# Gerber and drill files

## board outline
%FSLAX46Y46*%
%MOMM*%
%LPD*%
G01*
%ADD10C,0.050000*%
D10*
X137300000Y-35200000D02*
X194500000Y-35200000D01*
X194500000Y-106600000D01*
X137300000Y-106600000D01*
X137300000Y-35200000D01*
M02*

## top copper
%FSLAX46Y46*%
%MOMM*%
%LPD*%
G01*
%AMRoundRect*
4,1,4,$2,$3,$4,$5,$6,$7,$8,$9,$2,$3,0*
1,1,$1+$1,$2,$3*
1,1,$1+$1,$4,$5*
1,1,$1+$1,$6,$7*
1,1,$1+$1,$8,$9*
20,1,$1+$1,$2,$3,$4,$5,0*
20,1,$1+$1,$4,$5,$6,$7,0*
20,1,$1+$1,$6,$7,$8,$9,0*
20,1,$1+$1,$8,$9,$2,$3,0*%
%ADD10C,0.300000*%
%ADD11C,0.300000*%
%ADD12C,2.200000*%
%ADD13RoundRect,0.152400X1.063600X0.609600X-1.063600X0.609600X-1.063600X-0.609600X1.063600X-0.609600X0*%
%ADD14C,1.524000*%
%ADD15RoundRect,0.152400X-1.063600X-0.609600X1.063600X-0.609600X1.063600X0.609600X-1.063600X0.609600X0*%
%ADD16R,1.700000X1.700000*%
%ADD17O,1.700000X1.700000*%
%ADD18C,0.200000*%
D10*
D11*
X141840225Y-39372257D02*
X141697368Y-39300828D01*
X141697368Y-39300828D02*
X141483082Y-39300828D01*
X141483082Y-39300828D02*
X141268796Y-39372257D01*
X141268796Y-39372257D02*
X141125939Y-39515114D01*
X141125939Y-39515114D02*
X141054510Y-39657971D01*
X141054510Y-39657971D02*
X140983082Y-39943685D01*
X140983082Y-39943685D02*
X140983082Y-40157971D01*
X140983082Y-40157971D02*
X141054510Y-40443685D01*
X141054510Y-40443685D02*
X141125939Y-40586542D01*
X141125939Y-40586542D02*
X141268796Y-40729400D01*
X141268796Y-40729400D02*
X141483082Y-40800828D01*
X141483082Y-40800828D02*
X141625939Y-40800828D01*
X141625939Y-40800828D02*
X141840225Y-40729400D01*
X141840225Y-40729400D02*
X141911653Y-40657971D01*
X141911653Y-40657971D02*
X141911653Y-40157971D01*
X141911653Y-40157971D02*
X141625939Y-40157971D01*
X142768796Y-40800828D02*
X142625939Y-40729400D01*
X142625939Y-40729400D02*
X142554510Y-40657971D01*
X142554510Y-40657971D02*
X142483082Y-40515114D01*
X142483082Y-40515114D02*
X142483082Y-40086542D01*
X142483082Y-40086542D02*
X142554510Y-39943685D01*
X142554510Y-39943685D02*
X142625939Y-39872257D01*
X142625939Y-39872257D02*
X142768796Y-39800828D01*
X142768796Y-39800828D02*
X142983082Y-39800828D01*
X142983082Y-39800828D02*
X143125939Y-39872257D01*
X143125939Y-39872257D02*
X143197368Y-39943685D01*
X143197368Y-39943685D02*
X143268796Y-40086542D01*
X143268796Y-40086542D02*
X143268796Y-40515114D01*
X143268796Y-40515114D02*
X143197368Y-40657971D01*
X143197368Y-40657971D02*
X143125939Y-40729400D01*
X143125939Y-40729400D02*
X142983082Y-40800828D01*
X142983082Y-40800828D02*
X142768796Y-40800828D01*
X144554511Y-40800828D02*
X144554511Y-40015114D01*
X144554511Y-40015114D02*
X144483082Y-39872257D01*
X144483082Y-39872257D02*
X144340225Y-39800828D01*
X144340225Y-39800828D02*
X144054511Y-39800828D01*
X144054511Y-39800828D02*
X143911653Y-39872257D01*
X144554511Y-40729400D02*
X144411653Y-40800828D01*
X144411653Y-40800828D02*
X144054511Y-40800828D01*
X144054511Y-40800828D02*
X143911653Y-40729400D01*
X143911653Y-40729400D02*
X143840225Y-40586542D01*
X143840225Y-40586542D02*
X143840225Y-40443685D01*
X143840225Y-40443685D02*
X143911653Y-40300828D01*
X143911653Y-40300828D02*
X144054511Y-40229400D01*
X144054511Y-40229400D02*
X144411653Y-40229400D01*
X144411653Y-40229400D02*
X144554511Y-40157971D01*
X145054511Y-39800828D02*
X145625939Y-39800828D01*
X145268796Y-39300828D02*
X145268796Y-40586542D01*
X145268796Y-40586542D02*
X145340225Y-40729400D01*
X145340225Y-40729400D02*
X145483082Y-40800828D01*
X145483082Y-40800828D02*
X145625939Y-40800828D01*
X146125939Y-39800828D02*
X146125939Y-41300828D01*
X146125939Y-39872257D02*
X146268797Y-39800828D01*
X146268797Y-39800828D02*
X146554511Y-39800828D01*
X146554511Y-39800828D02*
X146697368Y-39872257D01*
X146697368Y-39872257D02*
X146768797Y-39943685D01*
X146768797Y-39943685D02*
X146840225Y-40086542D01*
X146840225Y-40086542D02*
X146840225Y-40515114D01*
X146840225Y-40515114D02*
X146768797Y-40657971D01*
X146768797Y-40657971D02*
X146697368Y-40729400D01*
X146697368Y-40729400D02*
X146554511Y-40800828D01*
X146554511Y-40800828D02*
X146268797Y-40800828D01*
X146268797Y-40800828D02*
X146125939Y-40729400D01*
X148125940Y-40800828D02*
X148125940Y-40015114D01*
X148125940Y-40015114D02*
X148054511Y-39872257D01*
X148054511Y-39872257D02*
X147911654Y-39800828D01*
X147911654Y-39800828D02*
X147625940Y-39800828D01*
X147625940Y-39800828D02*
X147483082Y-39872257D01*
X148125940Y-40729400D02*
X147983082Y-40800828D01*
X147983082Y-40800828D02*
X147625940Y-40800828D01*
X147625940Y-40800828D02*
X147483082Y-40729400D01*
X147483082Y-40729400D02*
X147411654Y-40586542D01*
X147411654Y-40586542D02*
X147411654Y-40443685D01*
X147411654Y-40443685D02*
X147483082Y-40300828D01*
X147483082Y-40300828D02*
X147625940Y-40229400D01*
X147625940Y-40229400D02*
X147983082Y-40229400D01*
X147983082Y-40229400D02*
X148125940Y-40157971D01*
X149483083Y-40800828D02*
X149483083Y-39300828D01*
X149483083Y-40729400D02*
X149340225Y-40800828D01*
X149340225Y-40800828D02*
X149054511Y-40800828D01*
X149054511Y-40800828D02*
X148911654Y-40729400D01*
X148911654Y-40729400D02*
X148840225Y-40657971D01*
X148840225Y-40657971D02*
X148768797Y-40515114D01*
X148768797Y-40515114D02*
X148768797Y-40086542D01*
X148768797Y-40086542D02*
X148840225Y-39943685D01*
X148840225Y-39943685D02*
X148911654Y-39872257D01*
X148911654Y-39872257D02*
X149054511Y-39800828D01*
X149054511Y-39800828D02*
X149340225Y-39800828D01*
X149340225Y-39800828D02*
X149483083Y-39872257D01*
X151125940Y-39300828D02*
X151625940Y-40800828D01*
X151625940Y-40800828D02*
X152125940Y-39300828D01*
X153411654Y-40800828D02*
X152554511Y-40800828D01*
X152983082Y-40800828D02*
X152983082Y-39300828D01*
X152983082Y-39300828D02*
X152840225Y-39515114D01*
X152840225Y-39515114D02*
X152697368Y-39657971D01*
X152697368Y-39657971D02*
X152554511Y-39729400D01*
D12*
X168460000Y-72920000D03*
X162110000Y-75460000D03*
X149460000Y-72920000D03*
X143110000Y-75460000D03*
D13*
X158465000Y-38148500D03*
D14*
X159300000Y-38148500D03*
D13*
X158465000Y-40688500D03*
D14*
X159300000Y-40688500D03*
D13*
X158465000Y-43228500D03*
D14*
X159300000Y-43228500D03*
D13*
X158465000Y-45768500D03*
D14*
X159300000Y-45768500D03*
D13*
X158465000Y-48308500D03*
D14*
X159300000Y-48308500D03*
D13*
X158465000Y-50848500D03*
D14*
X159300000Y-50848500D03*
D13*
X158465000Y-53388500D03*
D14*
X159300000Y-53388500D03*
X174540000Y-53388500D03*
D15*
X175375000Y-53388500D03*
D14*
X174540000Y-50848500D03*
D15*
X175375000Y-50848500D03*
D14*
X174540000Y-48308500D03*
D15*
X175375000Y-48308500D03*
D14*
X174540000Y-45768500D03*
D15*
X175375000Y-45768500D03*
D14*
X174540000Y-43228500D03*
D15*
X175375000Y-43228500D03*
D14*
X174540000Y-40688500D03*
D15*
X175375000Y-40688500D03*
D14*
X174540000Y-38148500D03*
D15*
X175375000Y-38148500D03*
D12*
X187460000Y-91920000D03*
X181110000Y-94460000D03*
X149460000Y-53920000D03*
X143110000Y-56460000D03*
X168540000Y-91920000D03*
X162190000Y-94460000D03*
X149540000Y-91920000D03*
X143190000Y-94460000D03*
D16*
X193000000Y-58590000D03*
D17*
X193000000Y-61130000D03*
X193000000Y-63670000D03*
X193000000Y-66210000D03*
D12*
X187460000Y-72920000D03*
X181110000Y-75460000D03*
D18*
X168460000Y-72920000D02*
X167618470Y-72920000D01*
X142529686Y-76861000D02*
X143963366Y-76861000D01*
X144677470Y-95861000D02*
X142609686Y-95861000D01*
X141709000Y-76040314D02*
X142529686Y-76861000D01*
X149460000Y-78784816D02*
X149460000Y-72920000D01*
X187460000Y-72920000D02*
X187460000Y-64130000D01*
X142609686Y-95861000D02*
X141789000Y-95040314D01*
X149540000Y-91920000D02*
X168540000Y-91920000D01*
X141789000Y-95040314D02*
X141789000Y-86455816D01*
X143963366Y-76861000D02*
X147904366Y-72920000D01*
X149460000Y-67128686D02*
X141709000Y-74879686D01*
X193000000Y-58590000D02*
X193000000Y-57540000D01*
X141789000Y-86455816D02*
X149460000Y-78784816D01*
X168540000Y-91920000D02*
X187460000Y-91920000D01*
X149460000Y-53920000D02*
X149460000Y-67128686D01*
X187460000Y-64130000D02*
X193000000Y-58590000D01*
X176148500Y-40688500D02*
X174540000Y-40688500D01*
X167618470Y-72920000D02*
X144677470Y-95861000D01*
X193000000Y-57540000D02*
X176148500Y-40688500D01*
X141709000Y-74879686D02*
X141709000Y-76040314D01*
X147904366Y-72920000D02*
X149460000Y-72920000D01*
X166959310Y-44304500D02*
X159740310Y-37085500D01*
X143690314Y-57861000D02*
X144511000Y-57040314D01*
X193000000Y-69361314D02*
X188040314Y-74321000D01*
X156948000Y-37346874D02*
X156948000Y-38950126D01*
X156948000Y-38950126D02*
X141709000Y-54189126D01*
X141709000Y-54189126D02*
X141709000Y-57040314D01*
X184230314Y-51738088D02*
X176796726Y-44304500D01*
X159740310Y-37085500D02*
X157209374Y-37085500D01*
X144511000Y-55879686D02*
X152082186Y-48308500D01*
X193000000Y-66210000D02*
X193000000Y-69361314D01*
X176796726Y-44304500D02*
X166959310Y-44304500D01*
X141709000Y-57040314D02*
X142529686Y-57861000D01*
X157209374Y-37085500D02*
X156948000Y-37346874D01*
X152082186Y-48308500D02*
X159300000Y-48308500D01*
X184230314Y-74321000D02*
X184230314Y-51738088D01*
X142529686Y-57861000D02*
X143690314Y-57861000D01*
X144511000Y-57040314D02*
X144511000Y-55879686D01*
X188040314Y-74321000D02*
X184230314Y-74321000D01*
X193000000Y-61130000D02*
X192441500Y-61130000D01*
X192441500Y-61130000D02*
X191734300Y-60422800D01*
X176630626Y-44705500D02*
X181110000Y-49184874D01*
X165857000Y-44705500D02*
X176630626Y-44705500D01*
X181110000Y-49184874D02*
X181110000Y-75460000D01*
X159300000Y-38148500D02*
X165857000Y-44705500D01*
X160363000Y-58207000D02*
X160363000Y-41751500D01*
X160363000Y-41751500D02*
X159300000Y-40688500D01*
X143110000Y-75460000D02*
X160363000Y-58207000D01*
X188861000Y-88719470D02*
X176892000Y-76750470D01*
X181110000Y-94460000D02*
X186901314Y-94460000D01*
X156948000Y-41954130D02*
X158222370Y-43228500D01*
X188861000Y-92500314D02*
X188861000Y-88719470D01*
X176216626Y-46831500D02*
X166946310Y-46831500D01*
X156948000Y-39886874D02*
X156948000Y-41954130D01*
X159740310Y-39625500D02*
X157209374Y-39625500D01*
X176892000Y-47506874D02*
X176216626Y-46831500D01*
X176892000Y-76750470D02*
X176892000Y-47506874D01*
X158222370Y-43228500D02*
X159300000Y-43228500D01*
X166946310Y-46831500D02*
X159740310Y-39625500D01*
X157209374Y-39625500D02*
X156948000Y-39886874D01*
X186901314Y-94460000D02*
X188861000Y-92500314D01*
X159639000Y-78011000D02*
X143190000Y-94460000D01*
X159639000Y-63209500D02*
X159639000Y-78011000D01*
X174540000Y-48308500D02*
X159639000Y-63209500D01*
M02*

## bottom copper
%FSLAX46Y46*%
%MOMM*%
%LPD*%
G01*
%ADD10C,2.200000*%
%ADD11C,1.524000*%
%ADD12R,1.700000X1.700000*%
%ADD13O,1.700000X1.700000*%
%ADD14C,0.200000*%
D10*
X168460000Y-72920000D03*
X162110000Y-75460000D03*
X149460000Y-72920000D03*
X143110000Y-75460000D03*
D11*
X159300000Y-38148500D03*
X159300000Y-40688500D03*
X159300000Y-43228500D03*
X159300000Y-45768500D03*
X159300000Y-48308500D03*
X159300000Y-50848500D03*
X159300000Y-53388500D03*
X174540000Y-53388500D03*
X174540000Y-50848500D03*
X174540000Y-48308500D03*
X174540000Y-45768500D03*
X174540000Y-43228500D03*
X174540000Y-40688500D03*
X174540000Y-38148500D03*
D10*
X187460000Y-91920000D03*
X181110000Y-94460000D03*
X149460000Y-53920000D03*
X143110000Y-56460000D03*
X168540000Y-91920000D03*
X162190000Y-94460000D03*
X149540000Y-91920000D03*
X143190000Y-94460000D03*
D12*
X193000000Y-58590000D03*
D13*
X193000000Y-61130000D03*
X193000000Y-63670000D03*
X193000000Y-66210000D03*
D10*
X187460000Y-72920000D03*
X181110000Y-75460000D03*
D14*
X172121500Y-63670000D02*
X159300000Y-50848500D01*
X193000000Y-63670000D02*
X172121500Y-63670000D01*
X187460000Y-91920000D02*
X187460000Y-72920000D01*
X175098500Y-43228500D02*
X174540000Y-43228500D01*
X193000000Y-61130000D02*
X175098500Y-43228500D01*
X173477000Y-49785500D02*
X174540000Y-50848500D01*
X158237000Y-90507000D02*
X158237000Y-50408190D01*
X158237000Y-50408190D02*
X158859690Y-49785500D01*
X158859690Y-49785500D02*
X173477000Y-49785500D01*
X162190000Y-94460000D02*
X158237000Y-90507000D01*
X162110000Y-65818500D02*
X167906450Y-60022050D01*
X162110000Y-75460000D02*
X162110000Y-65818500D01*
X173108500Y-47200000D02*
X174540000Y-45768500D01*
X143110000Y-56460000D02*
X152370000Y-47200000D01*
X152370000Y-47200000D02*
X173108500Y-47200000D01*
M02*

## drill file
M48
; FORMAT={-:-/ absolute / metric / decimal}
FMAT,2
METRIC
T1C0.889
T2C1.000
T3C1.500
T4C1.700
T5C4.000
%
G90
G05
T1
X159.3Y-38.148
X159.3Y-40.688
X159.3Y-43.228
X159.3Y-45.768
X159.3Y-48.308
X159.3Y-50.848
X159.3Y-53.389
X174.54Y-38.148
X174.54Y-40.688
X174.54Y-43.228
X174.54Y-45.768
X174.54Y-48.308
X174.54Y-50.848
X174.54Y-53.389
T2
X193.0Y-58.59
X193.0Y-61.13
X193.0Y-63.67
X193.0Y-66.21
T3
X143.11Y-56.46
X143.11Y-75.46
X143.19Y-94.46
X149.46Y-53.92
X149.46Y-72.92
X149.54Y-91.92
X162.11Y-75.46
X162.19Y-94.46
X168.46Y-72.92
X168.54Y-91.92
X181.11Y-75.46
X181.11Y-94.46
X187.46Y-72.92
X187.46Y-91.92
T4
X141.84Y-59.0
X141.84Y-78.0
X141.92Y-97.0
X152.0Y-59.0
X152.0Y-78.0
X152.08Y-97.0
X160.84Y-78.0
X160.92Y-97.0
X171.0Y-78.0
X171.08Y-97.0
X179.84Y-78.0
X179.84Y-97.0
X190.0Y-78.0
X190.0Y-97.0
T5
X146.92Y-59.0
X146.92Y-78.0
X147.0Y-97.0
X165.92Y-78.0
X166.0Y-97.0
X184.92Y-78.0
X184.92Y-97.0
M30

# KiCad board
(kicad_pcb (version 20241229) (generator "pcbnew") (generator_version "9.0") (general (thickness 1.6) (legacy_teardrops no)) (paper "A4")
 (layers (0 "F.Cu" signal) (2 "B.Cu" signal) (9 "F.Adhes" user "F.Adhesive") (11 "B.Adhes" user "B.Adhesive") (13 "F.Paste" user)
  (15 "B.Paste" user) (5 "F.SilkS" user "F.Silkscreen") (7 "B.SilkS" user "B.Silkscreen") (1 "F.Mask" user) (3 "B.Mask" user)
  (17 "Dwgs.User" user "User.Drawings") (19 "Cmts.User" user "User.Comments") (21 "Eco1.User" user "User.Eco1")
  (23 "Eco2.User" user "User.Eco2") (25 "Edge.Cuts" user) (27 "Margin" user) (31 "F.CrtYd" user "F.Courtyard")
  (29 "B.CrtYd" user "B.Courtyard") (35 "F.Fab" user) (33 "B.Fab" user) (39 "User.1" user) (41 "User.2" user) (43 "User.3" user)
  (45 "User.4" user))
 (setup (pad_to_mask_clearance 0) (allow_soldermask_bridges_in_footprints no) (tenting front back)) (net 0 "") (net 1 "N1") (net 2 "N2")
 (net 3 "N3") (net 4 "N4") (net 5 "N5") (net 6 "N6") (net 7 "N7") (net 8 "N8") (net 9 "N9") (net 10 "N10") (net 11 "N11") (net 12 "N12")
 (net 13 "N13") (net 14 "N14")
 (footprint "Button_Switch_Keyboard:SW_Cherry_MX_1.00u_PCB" (layer "F.Cu") (at 168.46 72.92)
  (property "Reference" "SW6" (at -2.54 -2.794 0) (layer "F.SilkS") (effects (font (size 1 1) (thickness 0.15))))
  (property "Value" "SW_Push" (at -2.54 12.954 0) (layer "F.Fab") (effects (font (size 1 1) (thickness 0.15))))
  (pad "" np_thru_hole circle (at -7.62 5.08) (size 1.7 1.7) (drill 1.7) (layers "*.Cu" "*.Mask"))
  (pad "" np_thru_hole circle (at -2.54 5.08) (size 4 4) (drill 4) (layers "*.Cu" "*.Mask"))
  (pad "" np_thru_hole circle (at 2.54 5.08) (size 1.7 1.7) (drill 1.7) (layers "*.Cu" "*.Mask"))
  (pad "1" thru_hole circle (at 0 0) (size 2.2 2.2) (drill 1.5) (layers "*.Cu" "*.Mask") (remove_unused_layers no) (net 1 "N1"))
  (pad "2" thru_hole circle (at -6.35 2.54) (size 2.2 2.2) (drill 1.5) (layers "*.Cu" "*.Mask") (remove_unused_layers no) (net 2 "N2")))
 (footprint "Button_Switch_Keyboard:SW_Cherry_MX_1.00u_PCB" (layer "F.Cu") (at 149.46 72.92)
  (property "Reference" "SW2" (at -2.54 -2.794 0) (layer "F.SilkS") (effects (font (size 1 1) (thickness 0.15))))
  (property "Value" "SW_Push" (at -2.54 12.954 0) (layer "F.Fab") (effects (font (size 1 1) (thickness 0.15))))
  (pad "" np_thru_hole circle (at -7.62 5.08) (size 1.7 1.7) (drill 1.7) (layers "*.Cu" "*.Mask"))
  (pad "" np_thru_hole circle (at -2.54 5.08) (size 4 4) (drill 4) (layers "*.Cu" "*.Mask"))
  (pad "" np_thru_hole circle (at 2.54 5.08) (size 1.7 1.7) (drill 1.7) (layers "*.Cu" "*.Mask"))
  (pad "1" thru_hole circle (at 0 0) (size 2.2 2.2) (drill 1.5) (layers "*.Cu" "*.Mask") (remove_unused_layers no) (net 1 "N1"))
  (pad "2" thru_hole circle (at -6.35 2.54) (size 2.2 2.2) (drill 1.5) (layers "*.Cu" "*.Mask") (remove_unused_layers no) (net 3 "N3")))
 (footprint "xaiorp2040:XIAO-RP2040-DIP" (layer "F.Cu") (at 166.92 45.7685)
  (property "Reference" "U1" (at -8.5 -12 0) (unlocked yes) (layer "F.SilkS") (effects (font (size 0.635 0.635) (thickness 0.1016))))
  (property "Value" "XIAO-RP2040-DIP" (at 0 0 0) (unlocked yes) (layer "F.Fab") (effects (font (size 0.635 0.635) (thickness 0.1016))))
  (pad "1" smd roundrect (at -8.455 -7.62 180) (size 2.432 1.524) (layers "F.Cu" "F.Mask") (roundrect_rratio 0.1) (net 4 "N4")
   (thermal_bridge_angle 45))
  (pad "1" thru_hole circle (at -7.62 -7.62 180) (size 1.524 1.524) (drill 0.889) (layers "*.Cu" "*.Mask") (remove_unused_layers no)
   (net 4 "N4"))
  (pad "2" smd roundrect (at -8.455 -5.08 180) (size 2.432 1.524) (layers "F.Cu" "F.Mask") (roundrect_rratio 0.1) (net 3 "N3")
   (thermal_bridge_angle 45))
  (pad "2" thru_hole circle (at -7.62 -5.08 180) (size 1.524 1.524) (drill 0.889) (layers "*.Cu" "*.Mask") (remove_unused_layers no)
   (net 3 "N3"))
  (pad "3" smd roundrect (at -8.455 -2.54 180) (size 2.432 1.524) (layers "F.Cu" "F.Mask") (roundrect_rratio 0.1) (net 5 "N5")
   (thermal_bridge_angle 45))
  (pad "3" thru_hole circle (at -7.62 -2.54 180) (size 1.524 1.524) (drill 0.889) (layers "*.Cu" "*.Mask") (remove_unused_layers no)
   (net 5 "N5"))
  (pad "4" smd roundrect (at -8.455 0 180) (size 2.432 1.524) (layers "F.Cu" "F.Mask") (roundrect_rratio 0.1) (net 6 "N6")
   (thermal_bridge_angle 45))
  (pad "4" thru_hole circle (at -7.62 0 180) (size 1.524 1.524) (drill 0.889) (layers "*.Cu" "*.Mask") (remove_unused_layers no)
   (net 6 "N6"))
  (pad "5" smd roundrect (at -8.455 2.54 180) (size 2.432 1.524) (layers "F.Cu" "F.Mask") (roundrect_rratio 0.1) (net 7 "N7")
   (thermal_bridge_angle 45))
  (pad "5" thru_hole circle (at -7.62 2.54 180) (size 1.524 1.524) (drill 0.889) (layers "*.Cu" "*.Mask") (remove_unused_layers no)
   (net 7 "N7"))
  (pad "6" smd roundrect (at -8.455 5.08 180) (size 2.432 1.524) (layers "F.Cu" "F.Mask") (roundrect_rratio 0.1) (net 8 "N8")
   (thermal_bridge_angle 45))
  (pad "6" thru_hole circle (at -7.62 5.08 180) (size 1.524 1.524) (drill 0.889) (layers "*.Cu" "*.Mask") (remove_unused_layers no)
   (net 8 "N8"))
  (pad "7" smd roundrect (at -8.455 7.62 180) (size 2.432 1.524) (layers "F.Cu" "F.Mask") (roundrect_rratio 0.1) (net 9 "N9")
   (thermal_bridge_angle 45))
  (pad "7" thru_hole circle (at -7.62 7.62 180) (size 1.524 1.524) (drill 0.889) (layers "*.Cu" "*.Mask") (remove_unused_layers no)
   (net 9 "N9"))
  (pad "8" thru_hole circle (at 7.62 7.62) (size 1.524 1.524) (drill 0.889) (layers "*.Cu" "*.Mask") (remove_unused_layers no) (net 2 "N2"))
  (pad "8" smd roundrect (at 8.455 7.62) (size 2.432 1.524) (layers "F.Cu" "F.Mask") (roundrect_rratio 0.1) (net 2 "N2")
   (thermal_bridge_angle 45))
  (pad "9" thru_hole circle (at 7.62 5.08) (size 1.524 1.524) (drill 0.889) (layers "*.Cu" "*.Mask") (remove_unused_layers no)
   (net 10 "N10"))
  (pad "9" smd roundrect (at 8.455 5.08) (size 2.432 1.524) (layers "F.Cu" "F.Mask") (roundrect_rratio 0.1) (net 10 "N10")
   (thermal_bridge_angle 45))
  (pad "10" thru_hole circle (at 7.62 2.54) (size 1.524 1.524) (drill 0.889) (layers "*.Cu" "*.Mask") (remove_unused_layers no)
   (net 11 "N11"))
  (pad "10" smd roundrect (at 8.455 2.54) (size 2.432 1.524) (layers "F.Cu" "F.Mask") (roundrect_rratio 0.1) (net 11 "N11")
   (thermal_bridge_angle 45))
  (pad "11" thru_hole circle (at 7.62 0) (size 1.524 1.524) (drill 0.889) (layers "*.Cu" "*.Mask") (remove_unused_layers no) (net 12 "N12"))
  (pad "11" smd roundrect (at 8.455 0) (size 2.432 1.524) (layers "F.Cu" "F.Mask") (roundrect_rratio 0.1) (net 12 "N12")
   (thermal_bridge_angle 45))
  (pad "12" thru_hole circle (at 7.62 -2.54) (size 1.524 1.524) (drill 0.889) (layers "*.Cu" "*.Mask") (remove_unused_layers no)
   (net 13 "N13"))
  (pad "12" smd roundrect (at 8.455 -2.54) (size 2.432 1.524) (layers "F.Cu" "F.Mask") (roundrect_rratio 0.1) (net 13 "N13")
   (thermal_bridge_angle 45))
  (pad "13" thru_hole circle (at 7.62 -5.08) (size 1.524 1.524) (drill 0.889) (layers "*.Cu" "*.Mask") (remove_unused_layers no)
   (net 1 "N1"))
  (pad "13" smd roundrect (at 8.455 -5.08) (size 2.432 1.524) (layers "F.Cu" "F.Mask") (roundrect_rratio 0.1) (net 1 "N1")
   (thermal_bridge_angle 45))
  (pad "14" thru_hole circle (at 7.62 -7.62) (size 1.524 1.524) (drill 0.889) (layers "*.Cu" "*.Mask") (remove_unused_layers no)
   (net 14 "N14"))
  (pad "14" smd roundrect (at 8.455 -7.62) (size 2.432 1.524) (layers "F.Cu" "F.Mask") (roundrect_rratio 0.1) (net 14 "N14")
   (thermal_bridge_angle 45)))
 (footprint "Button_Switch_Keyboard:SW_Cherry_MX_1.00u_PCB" (layer "F.Cu") (at 187.46 91.92)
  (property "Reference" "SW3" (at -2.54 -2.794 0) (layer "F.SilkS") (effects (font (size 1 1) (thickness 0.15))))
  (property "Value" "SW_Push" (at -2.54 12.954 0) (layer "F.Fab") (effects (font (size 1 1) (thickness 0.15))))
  (pad "" np_thru_hole circle (at -7.62 5.08) (size 1.7 1.7) (drill 1.7) (layers "*.Cu" "*.Mask"))
  (pad "" np_thru_hole circle (at -2.54 5.08) (size 4 4) (drill 4) (layers "*.Cu" "*.Mask"))
  (pad "" np_thru_hole circle (at 2.54 5.08) (size 1.7 1.7) (drill 1.7) (layers "*.Cu" "*.Mask"))
  (pad "1" thru_hole circle (at 0 0) (size 2.2 2.2) (drill 1.5) (layers "*.Cu" "*.Mask") (remove_unused_layers no) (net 1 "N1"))
  (pad "2" thru_hole circle (at -6.35 2.54) (size 2.2 2.2) (drill 1.5) (layers "*.Cu" "*.Mask") (remove_unused_layers no) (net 5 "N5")))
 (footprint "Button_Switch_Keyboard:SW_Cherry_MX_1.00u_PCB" (layer "F.Cu") (at 149.46 53.92)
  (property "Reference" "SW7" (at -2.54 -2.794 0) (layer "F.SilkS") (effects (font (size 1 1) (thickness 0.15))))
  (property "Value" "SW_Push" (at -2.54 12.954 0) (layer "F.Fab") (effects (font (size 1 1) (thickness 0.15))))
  (pad "" np_thru_hole circle (at -7.62 5.08) (size 1.7 1.7) (drill 1.7) (layers "*.Cu" "*.Mask"))
  (pad "" np_thru_hole circle (at -2.54 5.08) (size 4 4) (drill 4) (layers "*.Cu" "*.Mask"))
  (pad "" np_thru_hole circle (at 2.54 5.08) (size 1.7 1.7) (drill 1.7) (layers "*.Cu" "*.Mask"))
  (pad "1" thru_hole circle (at 0 0) (size 2.2 2.2) (drill 1.5) (layers "*.Cu" "*.Mask") (remove_unused_layers no) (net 1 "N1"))
  (pad "2" thru_hole circle (at -6.35 2.54) (size 2.2 2.2) (drill 1.5) (layers "*.Cu" "*.Mask") (remove_unused_layers no) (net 12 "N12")))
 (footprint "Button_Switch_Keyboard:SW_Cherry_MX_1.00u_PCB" (layer "F.Cu") (at 168.54 91.92)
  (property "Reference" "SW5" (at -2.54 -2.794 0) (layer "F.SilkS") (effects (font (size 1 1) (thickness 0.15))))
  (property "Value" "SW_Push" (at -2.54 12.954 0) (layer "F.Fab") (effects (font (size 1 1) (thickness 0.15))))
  (pad "" np_thru_hole circle (at -7.62 5.08) (size 1.7 1.7) (drill 1.7) (layers "*.Cu" "*.Mask"))
  (pad "" np_thru_hole circle (at -2.54 5.08) (size 4 4) (drill 4) (layers "*.Cu" "*.Mask"))
  (pad "" np_thru_hole circle (at 2.54 5.08) (size 1.7 1.7) (drill 1.7) (layers "*.Cu" "*.Mask"))
  (pad "1" thru_hole circle (at 0 0) (size 2.2 2.2) (drill 1.5) (layers "*.Cu" "*.Mask") (remove_unused_layers no) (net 1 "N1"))
  (pad "2" thru_hole circle (at -6.35 2.54) (size 2.2 2.2) (drill 1.5) (layers "*.Cu" "*.Mask") (remove_unused_layers no) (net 10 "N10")))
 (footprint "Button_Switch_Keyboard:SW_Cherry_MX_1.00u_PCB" (layer "F.Cu") (at 149.54 91.92)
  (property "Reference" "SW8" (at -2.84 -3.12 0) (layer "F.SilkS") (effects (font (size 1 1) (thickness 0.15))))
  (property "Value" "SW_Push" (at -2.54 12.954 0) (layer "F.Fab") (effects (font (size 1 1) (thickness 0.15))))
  (pad "" np_thru_hole circle (at -7.62 5.08) (size 1.7 1.7) (drill 1.7) (layers "*.Cu" "*.Mask"))
  (pad "" np_thru_hole circle (at -2.54 5.08) (size 4 4) (drill 4) (layers "*.Cu" "*.Mask"))
  (pad "" np_thru_hole circle (at 2.54 5.08) (size 1.7 1.7) (drill 1.7) (layers "*.Cu" "*.Mask"))
  (pad "1" thru_hole circle (at 0 0) (size 2.2 2.2) (drill 1.5) (layers "*.Cu" "*.Mask") (remove_unused_layers no) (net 1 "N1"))
  (pad "2" thru_hole circle (at -6.35 2.54) (size 2.2 2.2) (drill 1.5) (layers "*.Cu" "*.Mask") (remove_unused_layers no) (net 11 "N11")))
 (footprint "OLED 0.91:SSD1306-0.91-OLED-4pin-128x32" (layer "F.Cu") (at 156.5 56.4)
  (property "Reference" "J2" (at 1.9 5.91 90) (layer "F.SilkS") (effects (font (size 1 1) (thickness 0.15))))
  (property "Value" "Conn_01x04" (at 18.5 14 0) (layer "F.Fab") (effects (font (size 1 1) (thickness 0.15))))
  (pad "1" thru_hole rect (at 36.5 2.19) (size 1.7 1.7) (drill 1) (layers "*.Cu" "*.Mask") (remove_unused_layers no) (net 1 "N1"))
  (pad "2" thru_hole oval (at 36.5 4.73) (size 1.7 1.7) (drill 1) (layers "*.Cu" "*.Mask") (remove_unused_layers no) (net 13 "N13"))
  (pad "3" thru_hole oval (at 36.5 7.27) (size 1.7 1.7) (drill 1) (layers "*.Cu" "*.Mask") (remove_unused_layers no) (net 8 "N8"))
  (pad "4" thru_hole oval (at 36.5 9.81) (size 1.7 1.7) (drill 1) (layers "*.Cu" "*.Mask") (remove_unused_layers no) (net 7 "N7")))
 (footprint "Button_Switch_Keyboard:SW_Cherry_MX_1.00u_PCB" (layer "F.Cu") (at 187.46 72.92)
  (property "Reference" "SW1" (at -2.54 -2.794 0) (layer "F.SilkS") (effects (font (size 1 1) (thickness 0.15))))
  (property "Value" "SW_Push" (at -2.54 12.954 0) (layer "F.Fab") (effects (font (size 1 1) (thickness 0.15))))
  (pad "" np_thru_hole circle (at -7.62 5.08) (size 1.7 1.7) (drill 1.7) (layers "*.Cu" "*.Mask"))
  (pad "" np_thru_hole circle (at -2.54 5.08) (size 4 4) (drill 4) (layers "*.Cu" "*.Mask"))
  (pad "" np_thru_hole circle (at 2.54 5.08) (size 1.7 1.7) (drill 1.7) (layers "*.Cu" "*.Mask"))
  (pad "1" thru_hole circle (at 0 0) (size 2.2 2.2) (drill 1.5) (layers "*.Cu" "*.Mask") (remove_unused_layers no) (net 1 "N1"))
  (pad "2" thru_hole circle (at -6.35 2.54) (size 2.2 2.2) (drill 1.5) (layers "*.Cu" "*.Mask") (remove_unused_layers no) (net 4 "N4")))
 (gr_rect (start 137.3 35.2) (end 194.5 106.6) (stroke (width 0.05) (type default)) (fill no) (layer "Edge.Cuts"))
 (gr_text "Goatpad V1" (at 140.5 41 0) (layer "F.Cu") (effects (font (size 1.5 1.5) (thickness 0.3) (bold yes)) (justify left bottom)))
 (segment (start 172.1215 63.67) (end 159.3 50.8485) (width 0.2) (layer "B.Cu") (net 8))
 (segment (start 193 63.67) (end 172.1215 63.67) (width 0.2) (layer "B.Cu") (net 8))
 (segment (start 168.46 72.92) (end 167.61847 72.92) (width 0.2) (layer "F.Cu") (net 1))
 (segment (start 142.529686 76.861) (end 143.963366 76.861) (width 0.2) (layer "F.Cu") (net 1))
 (segment (start 144.67747 95.861) (end 142.609686 95.861) (width 0.2) (layer "F.Cu") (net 1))
 (segment (start 141.709 76.040314) (end 142.529686 76.861) (width 0.2) (layer "F.Cu") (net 1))
 (segment (start 149.46 78.784816) (end 149.46 72.92) (width 0.2) (layer "F.Cu") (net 1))
 (segment (start 187.46 72.92) (end 187.46 64.13) (width 0.2) (layer "F.Cu") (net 1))
 (segment (start 142.609686 95.861) (end 141.789 95.040314) (width 0.2) (layer "F.Cu") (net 1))
 (segment (start 149.54 91.92) (end 168.54 91.92) (width 0.2) (layer "F.Cu") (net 1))
 (segment (start 141.789 95.040314) (end 141.789 86.455816) (width 0.2) (layer "F.Cu") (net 1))
 (segment (start 143.963366 76.861) (end 147.904366 72.92) (width 0.2) (layer "F.Cu") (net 1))
 (segment (start 149.46 67.128686) (end 141.709 74.879686) (width 0.2) (layer "F.Cu") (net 1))
 (segment (start 193 58.59) (end 193 57.54) (width 0.2) (layer "F.Cu") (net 1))
 (segment (start 141.789 86.455816) (end 149.46 78.784816) (width 0.2) (layer "F.Cu") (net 1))
 (segment (start 168.54 91.92) (end 187.46 91.92) (width 0.2) (layer "F.Cu") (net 1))
 (segment (start 149.46 53.92) (end 149.46 67.128686) (width 0.2) (layer "F.Cu") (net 1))
 (segment (start 187.46 64.13) (end 193 58.59) (width 0.2) (layer "F.Cu") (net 1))
 (segment (start 176.1485 40.6885) (end 174.54 40.6885) (width 0.2) (layer "F.Cu") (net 1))
 (segment (start 167.61847 72.92) (end 144.67747 95.861) (width 0.2) (layer "F.Cu") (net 1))
 (segment (start 193 57.54) (end 176.1485 40.6885) (width 0.2) (layer "F.Cu") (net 1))
 (segment (start 141.709 74.879686) (end 141.709 76.040314) (width 0.2) (layer "F.Cu") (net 1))
 (segment (start 147.904366 72.92) (end 149.46 72.92) (width 0.2) (layer "F.Cu") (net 1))
 (segment (start 187.46 91.92) (end 187.46 72.92) (width 0.2) (layer "B.Cu") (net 1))
 (segment (start 166.95931 44.3045) (end 159.74031 37.0855) (width 0.2) (layer "F.Cu") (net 7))
 (segment (start 143.690314 57.861) (end 144.511 57.040314) (width 0.2) (layer "F.Cu") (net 7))
 (segment (start 193 69.361314) (end 188.040314 74.321) (width 0.2) (layer "F.Cu") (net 7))
 (segment (start 156.948 37.346874) (end 156.948 38.950126) (width 0.2) (layer "F.Cu") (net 7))
 (segment (start 156.948 38.950126) (end 141.709 54.189126) (width 0.2) (layer "F.Cu") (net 7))
 (segment (start 141.709 54.189126) (end 141.709 57.040314) (width 0.2) (layer "F.Cu") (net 7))
 (segment (start 184.230314 51.738088) (end 176.796726 44.3045) (width 0.2) (layer "F.Cu") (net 7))
 (segment (start 159.74031 37.0855) (end 157.209374 37.0855) (width 0.2) (layer "F.Cu") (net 7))
 (segment (start 144.511 55.879686) (end 152.082186 48.3085) (width 0.2) (layer "F.Cu") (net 7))
 (segment (start 193 66.21) (end 193 69.361314) (width 0.2) (layer "F.Cu") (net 7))
 (segment (start 176.796726 44.3045) (end 166.95931 44.3045) (width 0.2) (layer "F.Cu") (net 7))
 (segment (start 141.709 57.040314) (end 142.529686 57.861) (width 0.2) (layer "F.Cu") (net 7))
 (segment (start 157.209374 37.0855) (end 156.948 37.346874) (width 0.2) (layer "F.Cu") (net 7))
 (segment (start 152.082186 48.3085) (end 159.3 48.3085) (width 0.2) (layer "F.Cu") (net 7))
 (segment (start 184.230314 74.321) (end 184.230314 51.738088) (width 0.2) (layer "F.Cu") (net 7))
 (segment (start 142.529686 57.861) (end 143.690314 57.861) (width 0.2) (layer "F.Cu") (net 7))
 (segment (start 144.511 57.040314) (end 144.511 55.879686) (width 0.2) (layer "F.Cu") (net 7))
 (segment (start 188.040314 74.321) (end 184.230314 74.321) (width 0.2) (layer "F.Cu") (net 7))
 (segment (start 193 61.13) (end 192.4415 61.13) (width 0.2) (layer "F.Cu") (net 13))
 (segment (start 192.4415 61.13) (end 191.7343 60.4228) (width 0.2) (layer "F.Cu") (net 13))
 (segment (start 175.0985 43.2285) (end 174.54 43.2285) (width 0.2) (layer "B.Cu") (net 13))
 (segment (start 193 61.13) (end 175.0985 43.2285) (width 0.2) (layer "B.Cu") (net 13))
 (segment (start 176.630626 44.7055) (end 181.11 49.184874) (width 0.2) (layer "F.Cu") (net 4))
 (segment (start 165.857 44.7055) (end 176.630626 44.7055) (width 0.2) (layer "F.Cu") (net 4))
 (segment (start 181.11 49.184874) (end 181.11 75.46) (width 0.2) (layer "F.Cu") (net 4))
 (segment (start 159.3 38.1485) (end 165.857 44.7055) (width 0.2) (layer "F.Cu") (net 4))
 (segment (start 160.363 58.207) (end 160.363 41.7515) (width 0.2) (layer "F.Cu") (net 3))
 (segment (start 160.363 41.7515) (end 159.3 40.6885) (width 0.2) (layer "F.Cu") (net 3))
 (segment (start 143.11 75.46) (end 160.363 58.207) (width 0.2) (layer "F.Cu") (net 3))
 (segment (start 188.861 88.71947) (end 176.892 76.75047) (width 0.2) (layer "F.Cu") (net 5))
 (segment (start 181.11 94.46) (end 186.901314 94.46) (width 0.2) (layer "F.Cu") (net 5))
 (segment (start 156.948 41.95413) (end 158.22237 43.2285) (width 0.2) (layer "F.Cu") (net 5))
 (segment (start 188.861 92.500314) (end 188.861 88.71947) (width 0.2) (layer "F.Cu") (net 5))
 (segment (start 176.216626 46.8315) (end 166.94631 46.8315) (width 0.2) (layer "F.Cu") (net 5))
 (segment (start 156.948 39.886874) (end 156.948 41.95413) (width 0.2) (layer "F.Cu") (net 5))
 (segment (start 159.74031 39.6255) (end 157.209374 39.6255) (width 0.2) (layer "F.Cu") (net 5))
 (segment (start 176.892 47.506874) (end 176.216626 46.8315) (width 0.2) (layer "F.Cu") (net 5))
 (segment (start 176.892 76.75047) (end 176.892 47.506874) (width 0.2) (layer "F.Cu") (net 5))
 (segment (start 158.22237 43.2285) (end 159.3 43.2285) (width 0.2) (layer "F.Cu") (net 5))
 (segment (start 166.94631 46.8315) (end 159.74031 39.6255) (width 0.2) (layer "F.Cu") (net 5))
 (segment (start 157.209374 39.6255) (end 156.948 39.886874) (width 0.2) (layer "F.Cu") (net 5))
 (segment (start 186.901314 94.46) (end 188.861 92.500314) (width 0.2) (layer "F.Cu") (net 5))
 (segment (start 173.477 49.7855) (end 174.54 50.8485) (width 0.2) (layer "B.Cu") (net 10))
 (segment (start 158.237 90.507) (end 158.237 50.40819) (width 0.2) (layer "B.Cu") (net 10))
 (segment (start 158.237 50.40819) (end 158.85969 49.7855) (width 0.2) (layer "B.Cu") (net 10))
 (segment (start 158.85969 49.7855) (end 173.477 49.7855) (width 0.2) (layer "B.Cu") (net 10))
 (segment (start 162.19 94.46) (end 158.237 90.507) (width 0.2) (layer "B.Cu") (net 10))
 (segment (start 162.11 65.8185) (end 167.90645 60.02205) (width 0.2) (layer "B.Cu") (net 2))
 (segment (start 162.11 75.46) (end 162.11 65.8185) (width 0.2) (layer "B.Cu") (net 2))
 (segment (start 173.1085 47.2) (end 174.54 45.7685) (width 0.2) (layer "B.Cu") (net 12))
 (segment (start 143.11 56.46) (end 152.37 47.2) (width 0.2) (layer "B.Cu") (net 12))
 (segment (start 152.37 47.2) (end 173.1085 47.2) (width 0.2) (layer "B.Cu") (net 12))
 (segment (start 159.639 78.011) (end 143.19 94.46) (width 0.2) (layer "F.Cu") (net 11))
 (segment (start 159.639 63.2095) (end 159.639 78.011) (width 0.2) (layer "F.Cu") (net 11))
 (segment (start 174.54 48.3085) (end 159.639 63.2095) (width 0.2) (layer "F.Cu") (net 11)))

